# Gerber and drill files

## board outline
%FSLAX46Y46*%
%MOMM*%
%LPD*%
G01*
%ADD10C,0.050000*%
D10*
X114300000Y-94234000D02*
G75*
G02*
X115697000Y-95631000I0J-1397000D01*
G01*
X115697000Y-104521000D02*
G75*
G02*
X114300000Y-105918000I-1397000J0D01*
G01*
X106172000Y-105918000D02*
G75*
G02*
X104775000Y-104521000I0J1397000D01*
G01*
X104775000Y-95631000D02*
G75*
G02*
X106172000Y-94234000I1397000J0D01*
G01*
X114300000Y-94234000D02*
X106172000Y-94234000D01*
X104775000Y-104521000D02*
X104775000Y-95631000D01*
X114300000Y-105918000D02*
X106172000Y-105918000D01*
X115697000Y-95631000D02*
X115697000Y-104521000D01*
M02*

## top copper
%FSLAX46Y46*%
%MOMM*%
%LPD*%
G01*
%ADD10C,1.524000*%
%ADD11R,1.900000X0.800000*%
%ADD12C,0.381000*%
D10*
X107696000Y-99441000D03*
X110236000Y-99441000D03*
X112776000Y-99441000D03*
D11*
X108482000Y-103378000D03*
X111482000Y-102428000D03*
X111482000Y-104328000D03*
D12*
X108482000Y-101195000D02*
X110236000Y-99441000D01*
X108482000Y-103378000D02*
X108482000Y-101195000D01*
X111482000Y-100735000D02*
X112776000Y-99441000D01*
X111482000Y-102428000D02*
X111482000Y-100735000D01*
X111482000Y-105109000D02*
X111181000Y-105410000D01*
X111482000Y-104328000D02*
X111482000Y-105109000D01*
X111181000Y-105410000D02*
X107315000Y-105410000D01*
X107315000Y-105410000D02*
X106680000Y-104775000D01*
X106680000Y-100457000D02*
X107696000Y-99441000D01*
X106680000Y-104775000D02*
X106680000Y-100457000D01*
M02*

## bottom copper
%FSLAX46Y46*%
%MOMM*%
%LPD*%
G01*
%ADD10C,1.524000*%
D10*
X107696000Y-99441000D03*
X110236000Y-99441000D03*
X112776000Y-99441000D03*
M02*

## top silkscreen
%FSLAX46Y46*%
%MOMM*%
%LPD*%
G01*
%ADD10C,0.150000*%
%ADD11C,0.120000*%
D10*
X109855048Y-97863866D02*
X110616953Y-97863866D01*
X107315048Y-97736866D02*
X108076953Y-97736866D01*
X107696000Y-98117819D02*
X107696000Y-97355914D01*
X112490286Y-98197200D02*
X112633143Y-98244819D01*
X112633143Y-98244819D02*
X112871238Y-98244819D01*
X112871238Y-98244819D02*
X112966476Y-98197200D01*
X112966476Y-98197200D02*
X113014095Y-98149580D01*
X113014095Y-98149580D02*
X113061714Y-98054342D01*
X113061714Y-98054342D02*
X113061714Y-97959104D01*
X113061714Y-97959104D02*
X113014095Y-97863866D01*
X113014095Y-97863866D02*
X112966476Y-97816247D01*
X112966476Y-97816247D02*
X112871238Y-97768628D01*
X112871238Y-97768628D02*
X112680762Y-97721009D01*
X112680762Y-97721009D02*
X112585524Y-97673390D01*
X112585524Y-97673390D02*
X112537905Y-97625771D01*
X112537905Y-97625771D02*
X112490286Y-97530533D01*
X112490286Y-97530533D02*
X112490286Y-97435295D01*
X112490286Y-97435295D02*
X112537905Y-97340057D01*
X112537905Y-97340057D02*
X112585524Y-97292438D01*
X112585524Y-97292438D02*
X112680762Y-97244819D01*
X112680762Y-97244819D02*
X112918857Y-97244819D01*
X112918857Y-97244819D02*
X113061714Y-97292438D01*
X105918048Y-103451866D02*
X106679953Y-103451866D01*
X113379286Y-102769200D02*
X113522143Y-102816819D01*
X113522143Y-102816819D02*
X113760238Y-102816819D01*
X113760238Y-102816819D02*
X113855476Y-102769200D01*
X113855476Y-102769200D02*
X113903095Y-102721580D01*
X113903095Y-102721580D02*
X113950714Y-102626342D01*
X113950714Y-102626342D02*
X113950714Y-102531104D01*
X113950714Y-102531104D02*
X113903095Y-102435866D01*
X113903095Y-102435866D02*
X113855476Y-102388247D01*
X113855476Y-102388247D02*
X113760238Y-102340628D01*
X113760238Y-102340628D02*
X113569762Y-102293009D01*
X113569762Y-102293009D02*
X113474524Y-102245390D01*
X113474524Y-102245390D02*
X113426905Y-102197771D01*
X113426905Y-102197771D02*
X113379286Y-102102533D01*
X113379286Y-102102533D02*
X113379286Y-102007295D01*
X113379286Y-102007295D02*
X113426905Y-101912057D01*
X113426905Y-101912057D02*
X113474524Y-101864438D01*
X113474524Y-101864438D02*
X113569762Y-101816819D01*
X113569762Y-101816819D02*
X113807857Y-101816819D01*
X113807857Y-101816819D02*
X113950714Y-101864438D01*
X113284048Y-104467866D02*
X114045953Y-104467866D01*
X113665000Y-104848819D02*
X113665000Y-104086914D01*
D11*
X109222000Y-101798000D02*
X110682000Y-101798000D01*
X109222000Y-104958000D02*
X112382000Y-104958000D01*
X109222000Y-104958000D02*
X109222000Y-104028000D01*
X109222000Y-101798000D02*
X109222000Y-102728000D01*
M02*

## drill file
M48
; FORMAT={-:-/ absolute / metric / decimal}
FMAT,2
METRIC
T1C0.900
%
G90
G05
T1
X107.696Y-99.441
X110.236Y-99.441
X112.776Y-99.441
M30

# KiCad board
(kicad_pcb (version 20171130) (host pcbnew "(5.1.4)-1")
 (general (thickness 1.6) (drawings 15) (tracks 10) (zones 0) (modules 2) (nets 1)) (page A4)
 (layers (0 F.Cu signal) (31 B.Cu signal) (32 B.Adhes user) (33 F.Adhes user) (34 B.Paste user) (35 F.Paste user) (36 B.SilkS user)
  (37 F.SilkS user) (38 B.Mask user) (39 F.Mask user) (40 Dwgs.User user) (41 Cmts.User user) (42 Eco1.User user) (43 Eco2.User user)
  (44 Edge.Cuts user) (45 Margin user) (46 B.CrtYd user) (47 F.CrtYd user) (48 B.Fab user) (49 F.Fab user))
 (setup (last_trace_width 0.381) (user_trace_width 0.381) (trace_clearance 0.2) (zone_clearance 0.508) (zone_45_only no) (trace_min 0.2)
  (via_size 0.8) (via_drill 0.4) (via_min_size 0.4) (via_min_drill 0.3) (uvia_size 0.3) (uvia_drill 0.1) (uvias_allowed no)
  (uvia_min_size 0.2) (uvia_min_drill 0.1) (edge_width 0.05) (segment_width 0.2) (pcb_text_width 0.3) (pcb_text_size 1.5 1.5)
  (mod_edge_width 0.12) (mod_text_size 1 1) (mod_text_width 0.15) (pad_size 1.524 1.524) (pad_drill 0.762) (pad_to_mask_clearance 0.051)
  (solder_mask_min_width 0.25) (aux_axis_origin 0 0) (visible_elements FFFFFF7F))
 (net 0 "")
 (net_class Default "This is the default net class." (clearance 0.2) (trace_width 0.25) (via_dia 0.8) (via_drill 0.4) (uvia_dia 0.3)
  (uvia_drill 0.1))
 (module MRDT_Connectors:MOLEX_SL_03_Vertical (layer B.Cu) (at 112.776 99.441 180)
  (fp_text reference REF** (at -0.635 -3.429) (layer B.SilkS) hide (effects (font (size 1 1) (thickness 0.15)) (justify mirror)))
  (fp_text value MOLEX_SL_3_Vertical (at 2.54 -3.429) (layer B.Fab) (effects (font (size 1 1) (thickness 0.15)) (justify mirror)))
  (pad 3 thru_hole circle (at 5.08 0 180) (size 1.524 1.524) (drill 0.9) (layers *.Cu *.Mask))
  (pad 2 thru_hole circle (at 2.54 0 180) (size 1.524 1.524) (drill 0.9) (layers *.Cu *.Mask))
  (pad 1 thru_hole circle (at 0 0 180) (size 1.524 1.524) (drill 0.9) (layers *.Cu *.Mask)))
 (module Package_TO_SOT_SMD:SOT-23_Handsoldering (layer F.Cu) (at 109.982 103.378 180)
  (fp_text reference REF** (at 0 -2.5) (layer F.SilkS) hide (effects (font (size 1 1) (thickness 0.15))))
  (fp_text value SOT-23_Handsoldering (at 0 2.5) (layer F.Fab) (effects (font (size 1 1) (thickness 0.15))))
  (fp_line (start 0.76 1.58) (end -0.7 1.58) (layer F.SilkS) (width 0.12))
  (fp_line (start 0.76 -1.58) (end -2.4 -1.58) (layer F.SilkS) (width 0.12))
  (fp_line (start 0.76 -1.58) (end 0.76 -0.65) (layer F.SilkS) (width 0.12))
  (fp_line (start 0.76 1.58) (end 0.76 0.65) (layer F.SilkS) (width 0.12))
  (pad 3 smd rect (at 1.5 0 180) (size 1.9 0.8) (layers F.Cu F.Paste F.Mask))
  (pad 2 smd rect (at -1.5 0.95 180) (size 1.9 0.8) (layers F.Cu F.Paste F.Mask))
  (pad 1 smd rect (at -1.5 -0.95 180) (size 1.9 0.8) (layers F.Cu F.Paste F.Mask)))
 (gr_arc (start 114.3 95.631) (end 115.697 95.631) (angle -90) (layer Edge.Cuts) (width 0.05))
 (gr_arc (start 114.3 104.521) (end 114.3 105.918) (angle -90) (layer Edge.Cuts) (width 0.05))
 (gr_arc (start 106.172 104.521) (end 104.775 104.521) (angle -90) (layer Edge.Cuts) (width 0.05))
 (gr_arc (start 106.172 95.631) (end 106.172 94.234) (angle -90) (layer Edge.Cuts) (width 0.05))
 (gr_line (start 114.3 94.234) (end 106.172 94.234) (layer Edge.Cuts) (width 0.05))
 (gr_line (start 104.775 104.521) (end 104.775 95.631) (layer Edge.Cuts) (width 0.05))
 (gr_line (start 114.3 105.918) (end 106.172 105.918) (layer Edge.Cuts) (width 0.05))
 (gr_line (start 115.697 95.631) (end 115.697 104.521) (layer Edge.Cuts) (width 0.05))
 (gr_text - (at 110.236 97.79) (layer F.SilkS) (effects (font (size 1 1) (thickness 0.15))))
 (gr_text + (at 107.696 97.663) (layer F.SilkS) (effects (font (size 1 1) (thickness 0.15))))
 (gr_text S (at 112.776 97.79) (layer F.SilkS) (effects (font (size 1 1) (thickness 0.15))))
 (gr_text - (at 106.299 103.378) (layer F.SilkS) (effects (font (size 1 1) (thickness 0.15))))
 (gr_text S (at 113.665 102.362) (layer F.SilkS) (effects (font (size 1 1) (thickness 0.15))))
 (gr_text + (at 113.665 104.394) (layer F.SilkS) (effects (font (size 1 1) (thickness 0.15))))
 (segment (start 108.482 101.195) (end 110.236 99.441) (width 0.381) (layer F.Cu) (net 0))
 (segment (start 108.482 103.378) (end 108.482 101.195) (width 0.381) (layer F.Cu) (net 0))
 (segment (start 111.482 100.735) (end 112.776 99.441) (width 0.381) (layer F.Cu) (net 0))
 (segment (start 111.482 102.428) (end 111.482 100.735) (width 0.381) (layer F.Cu) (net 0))
 (segment (start 111.482 105.109) (end 111.181 105.41) (width 0.381) (layer F.Cu) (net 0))
 (segment (start 111.482 104.328) (end 111.482 105.109) (width 0.381) (layer F.Cu) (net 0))
 (segment (start 111.181 105.41) (end 107.315 105.41) (width 0.381) (layer F.Cu) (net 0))
 (segment (start 107.315 105.41) (end 106.68 104.775) (width 0.381) (layer F.Cu) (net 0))
 (segment (start 106.68 100.457) (end 107.696 99.441) (width 0.381) (layer F.Cu) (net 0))
 (segment (start 106.68 104.775) (end 106.68 100.457) (width 0.381) (layer F.Cu) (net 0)))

